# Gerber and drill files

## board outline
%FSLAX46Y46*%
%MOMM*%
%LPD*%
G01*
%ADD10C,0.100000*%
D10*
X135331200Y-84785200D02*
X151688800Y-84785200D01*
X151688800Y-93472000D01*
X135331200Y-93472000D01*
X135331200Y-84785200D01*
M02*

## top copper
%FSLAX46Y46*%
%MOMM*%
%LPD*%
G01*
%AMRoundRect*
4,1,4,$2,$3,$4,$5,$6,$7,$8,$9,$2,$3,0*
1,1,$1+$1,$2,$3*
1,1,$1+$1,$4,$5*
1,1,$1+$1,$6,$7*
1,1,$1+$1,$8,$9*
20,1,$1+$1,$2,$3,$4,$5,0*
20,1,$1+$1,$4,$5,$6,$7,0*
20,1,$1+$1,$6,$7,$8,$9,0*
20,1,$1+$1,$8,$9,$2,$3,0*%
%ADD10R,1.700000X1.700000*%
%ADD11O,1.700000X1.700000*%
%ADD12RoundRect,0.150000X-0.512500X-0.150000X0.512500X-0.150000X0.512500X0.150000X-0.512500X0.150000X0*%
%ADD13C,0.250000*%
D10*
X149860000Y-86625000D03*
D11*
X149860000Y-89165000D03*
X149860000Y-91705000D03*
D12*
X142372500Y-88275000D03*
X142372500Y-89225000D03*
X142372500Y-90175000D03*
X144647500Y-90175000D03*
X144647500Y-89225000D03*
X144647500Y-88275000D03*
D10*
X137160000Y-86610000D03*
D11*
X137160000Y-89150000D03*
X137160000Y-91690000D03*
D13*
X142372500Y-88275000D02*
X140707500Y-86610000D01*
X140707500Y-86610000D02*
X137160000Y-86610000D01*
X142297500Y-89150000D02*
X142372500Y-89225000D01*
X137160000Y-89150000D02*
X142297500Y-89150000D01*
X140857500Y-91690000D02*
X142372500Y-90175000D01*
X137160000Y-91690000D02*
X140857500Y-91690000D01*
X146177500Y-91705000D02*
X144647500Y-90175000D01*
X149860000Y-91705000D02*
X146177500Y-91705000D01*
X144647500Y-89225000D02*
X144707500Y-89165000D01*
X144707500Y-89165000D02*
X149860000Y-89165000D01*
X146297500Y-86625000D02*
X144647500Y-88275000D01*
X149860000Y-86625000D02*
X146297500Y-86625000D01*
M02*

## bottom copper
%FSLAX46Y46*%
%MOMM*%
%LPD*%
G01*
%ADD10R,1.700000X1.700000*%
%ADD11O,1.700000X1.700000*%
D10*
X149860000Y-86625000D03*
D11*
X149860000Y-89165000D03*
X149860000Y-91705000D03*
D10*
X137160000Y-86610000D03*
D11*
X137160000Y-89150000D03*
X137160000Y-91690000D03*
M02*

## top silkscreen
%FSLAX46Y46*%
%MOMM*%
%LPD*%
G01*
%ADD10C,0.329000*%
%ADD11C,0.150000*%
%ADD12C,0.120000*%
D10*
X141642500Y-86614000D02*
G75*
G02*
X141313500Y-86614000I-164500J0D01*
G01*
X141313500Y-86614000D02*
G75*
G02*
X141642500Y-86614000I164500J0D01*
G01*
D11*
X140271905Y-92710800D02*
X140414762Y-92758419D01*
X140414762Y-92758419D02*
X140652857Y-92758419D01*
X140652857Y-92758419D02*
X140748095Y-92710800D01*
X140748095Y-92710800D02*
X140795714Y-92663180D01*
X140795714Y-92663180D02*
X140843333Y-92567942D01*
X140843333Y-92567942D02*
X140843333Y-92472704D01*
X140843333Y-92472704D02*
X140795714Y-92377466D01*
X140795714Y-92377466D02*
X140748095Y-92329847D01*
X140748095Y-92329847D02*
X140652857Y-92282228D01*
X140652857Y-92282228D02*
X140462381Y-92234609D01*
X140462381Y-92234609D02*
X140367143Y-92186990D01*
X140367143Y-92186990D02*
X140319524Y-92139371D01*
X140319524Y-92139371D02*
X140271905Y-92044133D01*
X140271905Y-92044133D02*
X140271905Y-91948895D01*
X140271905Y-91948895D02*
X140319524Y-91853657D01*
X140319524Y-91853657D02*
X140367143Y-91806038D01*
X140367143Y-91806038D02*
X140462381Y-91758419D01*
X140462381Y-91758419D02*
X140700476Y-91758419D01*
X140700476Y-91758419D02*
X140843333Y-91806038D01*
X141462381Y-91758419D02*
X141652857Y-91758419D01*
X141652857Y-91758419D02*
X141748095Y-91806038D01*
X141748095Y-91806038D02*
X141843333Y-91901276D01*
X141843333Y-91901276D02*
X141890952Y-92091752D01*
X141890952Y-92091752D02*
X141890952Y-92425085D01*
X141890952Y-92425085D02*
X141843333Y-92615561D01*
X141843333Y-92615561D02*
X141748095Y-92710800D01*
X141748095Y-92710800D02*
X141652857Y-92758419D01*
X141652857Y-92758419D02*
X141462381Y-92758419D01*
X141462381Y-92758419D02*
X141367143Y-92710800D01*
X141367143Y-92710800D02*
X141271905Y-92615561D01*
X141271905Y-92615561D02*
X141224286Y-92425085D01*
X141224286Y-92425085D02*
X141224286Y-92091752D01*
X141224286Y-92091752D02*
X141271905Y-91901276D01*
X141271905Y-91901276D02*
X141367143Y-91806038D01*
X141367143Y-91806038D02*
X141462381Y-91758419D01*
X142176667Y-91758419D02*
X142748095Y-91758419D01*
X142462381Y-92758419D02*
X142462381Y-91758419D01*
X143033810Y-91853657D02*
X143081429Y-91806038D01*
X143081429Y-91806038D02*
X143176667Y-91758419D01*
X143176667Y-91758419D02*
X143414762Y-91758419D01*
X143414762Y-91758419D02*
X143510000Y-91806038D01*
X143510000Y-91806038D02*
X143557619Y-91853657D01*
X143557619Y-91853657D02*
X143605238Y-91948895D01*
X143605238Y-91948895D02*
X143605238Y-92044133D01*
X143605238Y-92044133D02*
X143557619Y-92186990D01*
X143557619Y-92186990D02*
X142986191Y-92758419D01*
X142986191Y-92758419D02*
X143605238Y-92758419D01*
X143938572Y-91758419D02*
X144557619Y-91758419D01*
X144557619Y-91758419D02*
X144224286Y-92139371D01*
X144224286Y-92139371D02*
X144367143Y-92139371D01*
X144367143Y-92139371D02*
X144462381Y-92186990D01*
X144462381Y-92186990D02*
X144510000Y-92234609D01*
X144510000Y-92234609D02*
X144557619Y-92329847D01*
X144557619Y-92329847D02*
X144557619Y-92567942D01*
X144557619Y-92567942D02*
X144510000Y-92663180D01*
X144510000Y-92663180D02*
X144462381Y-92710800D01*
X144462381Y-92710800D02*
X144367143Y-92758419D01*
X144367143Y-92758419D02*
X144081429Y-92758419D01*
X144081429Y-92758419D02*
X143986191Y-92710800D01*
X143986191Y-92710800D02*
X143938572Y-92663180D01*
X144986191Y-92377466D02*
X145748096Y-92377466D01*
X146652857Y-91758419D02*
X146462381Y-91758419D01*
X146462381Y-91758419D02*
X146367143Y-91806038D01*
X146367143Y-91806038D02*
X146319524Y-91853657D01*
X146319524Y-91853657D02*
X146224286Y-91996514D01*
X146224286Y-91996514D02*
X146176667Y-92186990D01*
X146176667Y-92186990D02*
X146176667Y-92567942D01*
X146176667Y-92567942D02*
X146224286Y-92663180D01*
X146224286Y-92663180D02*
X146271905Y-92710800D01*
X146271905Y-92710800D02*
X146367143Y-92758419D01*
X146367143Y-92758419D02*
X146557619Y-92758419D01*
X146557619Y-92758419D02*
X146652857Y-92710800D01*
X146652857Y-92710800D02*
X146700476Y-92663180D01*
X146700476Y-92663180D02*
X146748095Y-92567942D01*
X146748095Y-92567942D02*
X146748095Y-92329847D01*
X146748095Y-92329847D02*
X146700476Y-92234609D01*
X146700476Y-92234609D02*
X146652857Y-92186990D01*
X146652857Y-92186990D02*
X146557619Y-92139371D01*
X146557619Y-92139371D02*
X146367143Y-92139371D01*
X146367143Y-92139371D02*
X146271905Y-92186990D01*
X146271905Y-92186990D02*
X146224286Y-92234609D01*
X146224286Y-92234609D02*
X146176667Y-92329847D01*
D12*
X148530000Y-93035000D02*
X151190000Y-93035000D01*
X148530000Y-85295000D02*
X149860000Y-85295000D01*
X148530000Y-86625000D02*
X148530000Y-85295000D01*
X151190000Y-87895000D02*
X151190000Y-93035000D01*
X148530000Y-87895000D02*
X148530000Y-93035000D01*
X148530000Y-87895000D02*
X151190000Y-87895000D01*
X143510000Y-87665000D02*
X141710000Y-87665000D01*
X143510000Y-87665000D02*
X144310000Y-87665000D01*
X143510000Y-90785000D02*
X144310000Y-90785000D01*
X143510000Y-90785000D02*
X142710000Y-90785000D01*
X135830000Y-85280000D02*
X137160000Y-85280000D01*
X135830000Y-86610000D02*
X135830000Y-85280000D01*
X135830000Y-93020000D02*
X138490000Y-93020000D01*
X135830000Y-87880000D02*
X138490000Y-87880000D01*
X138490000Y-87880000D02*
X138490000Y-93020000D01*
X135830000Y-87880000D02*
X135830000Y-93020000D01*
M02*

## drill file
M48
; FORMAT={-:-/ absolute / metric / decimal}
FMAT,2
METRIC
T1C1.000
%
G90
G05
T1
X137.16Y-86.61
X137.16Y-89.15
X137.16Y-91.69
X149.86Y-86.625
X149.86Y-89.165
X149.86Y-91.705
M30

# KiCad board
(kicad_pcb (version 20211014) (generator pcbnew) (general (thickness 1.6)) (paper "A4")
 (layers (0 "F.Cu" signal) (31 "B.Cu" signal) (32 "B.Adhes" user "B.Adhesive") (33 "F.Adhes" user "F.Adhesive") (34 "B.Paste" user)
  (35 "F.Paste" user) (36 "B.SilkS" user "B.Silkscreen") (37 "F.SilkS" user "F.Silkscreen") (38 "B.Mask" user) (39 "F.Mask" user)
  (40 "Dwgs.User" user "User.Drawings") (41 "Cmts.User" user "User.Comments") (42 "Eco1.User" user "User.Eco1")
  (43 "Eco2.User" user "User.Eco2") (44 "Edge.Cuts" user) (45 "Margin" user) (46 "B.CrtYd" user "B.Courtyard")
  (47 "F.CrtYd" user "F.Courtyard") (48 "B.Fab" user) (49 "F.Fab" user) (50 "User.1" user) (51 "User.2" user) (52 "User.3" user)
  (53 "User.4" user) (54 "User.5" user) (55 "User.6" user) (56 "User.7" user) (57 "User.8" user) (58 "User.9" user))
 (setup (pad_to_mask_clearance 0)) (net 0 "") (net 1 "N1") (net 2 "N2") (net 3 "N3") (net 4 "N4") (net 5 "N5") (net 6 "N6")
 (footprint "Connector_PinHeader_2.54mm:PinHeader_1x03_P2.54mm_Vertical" (layer "F.Cu") (at 149.86 86.625)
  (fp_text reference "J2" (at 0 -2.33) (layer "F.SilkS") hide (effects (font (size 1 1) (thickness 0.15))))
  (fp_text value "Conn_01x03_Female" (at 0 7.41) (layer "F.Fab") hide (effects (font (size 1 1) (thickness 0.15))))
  (fp_line (start -1.33 6.41) (end 1.33 6.41) (layer "F.SilkS") (width 0.12))
  (fp_line (start -1.33 -1.33) (end 0 -1.33) (layer "F.SilkS") (width 0.12))
  (fp_line (start -1.33 0) (end -1.33 -1.33) (layer "F.SilkS") (width 0.12))
  (fp_line (start 1.33 1.27) (end 1.33 6.41) (layer "F.SilkS") (width 0.12))
  (fp_line (start -1.33 1.27) (end -1.33 6.41) (layer "F.SilkS") (width 0.12))
  (fp_line (start -1.33 1.27) (end 1.33 1.27) (layer "F.SilkS") (width 0.12))
  (pad "1" thru_hole rect (at 0 0) (size 1.7 1.7) (drill 1) (layers *.Cu *.Mask) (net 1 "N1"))
  (pad "2" thru_hole oval (at 0 2.54) (size 1.7 1.7) (drill 1) (layers *.Cu *.Mask) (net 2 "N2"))
  (pad "3" thru_hole oval (at 0 5.08) (size 1.7 1.7) (drill 1) (layers *.Cu *.Mask) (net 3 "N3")))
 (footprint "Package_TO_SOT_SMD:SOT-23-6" (layer "F.Cu") (at 143.51 89.225)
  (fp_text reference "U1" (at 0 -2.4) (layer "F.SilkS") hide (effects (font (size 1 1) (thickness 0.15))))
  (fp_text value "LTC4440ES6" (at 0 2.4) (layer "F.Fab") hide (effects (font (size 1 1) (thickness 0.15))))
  (fp_line (start 0 -1.56) (end -1.8 -1.56) (layer "F.SilkS") (width 0.12))
  (fp_line (start 0 -1.56) (end 0.8 -1.56) (layer "F.SilkS") (width 0.12))
  (fp_line (start 0 1.56) (end 0.8 1.56) (layer "F.SilkS") (width 0.12))
  (fp_line (start 0 1.56) (end -0.8 1.56) (layer "F.SilkS") (width 0.12))
  (pad "1" smd roundrect (at -1.1375 -0.95) (size 1.325 0.6) (layers "F.Cu" "F.Paste" "F.Mask") (roundrect_rratio 0.25) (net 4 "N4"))
  (pad "2" smd roundrect (at -1.1375 0) (size 1.325 0.6) (layers "F.Cu" "F.Paste" "F.Mask") (roundrect_rratio 0.25) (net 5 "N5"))
  (pad "3" smd roundrect (at -1.1375 0.95) (size 1.325 0.6) (layers "F.Cu" "F.Paste" "F.Mask") (roundrect_rratio 0.25) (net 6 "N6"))
  (pad "4" smd roundrect (at 1.1375 0.95) (size 1.325 0.6) (layers "F.Cu" "F.Paste" "F.Mask") (roundrect_rratio 0.25) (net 3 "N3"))
  (pad "5" smd roundrect (at 1.1375 0) (size 1.325 0.6) (layers "F.Cu" "F.Paste" "F.Mask") (roundrect_rratio 0.25) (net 2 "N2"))
  (pad "6" smd roundrect (at 1.1375 -0.95) (size 1.325 0.6) (layers "F.Cu" "F.Paste" "F.Mask") (roundrect_rratio 0.25) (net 1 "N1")))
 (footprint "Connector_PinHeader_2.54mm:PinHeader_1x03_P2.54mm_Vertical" (layer "F.Cu") (at 137.16 86.61)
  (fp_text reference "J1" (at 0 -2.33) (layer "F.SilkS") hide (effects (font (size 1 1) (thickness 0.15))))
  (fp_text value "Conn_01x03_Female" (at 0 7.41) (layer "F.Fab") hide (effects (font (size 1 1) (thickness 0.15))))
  (fp_line (start -1.33 -1.33) (end 0 -1.33) (layer "F.SilkS") (width 0.12))
  (fp_line (start -1.33 0) (end -1.33 -1.33) (layer "F.SilkS") (width 0.12))
  (fp_line (start -1.33 6.41) (end 1.33 6.41) (layer "F.SilkS") (width 0.12))
  (fp_line (start -1.33 1.27) (end 1.33 1.27) (layer "F.SilkS") (width 0.12))
  (fp_line (start 1.33 1.27) (end 1.33 6.41) (layer "F.SilkS") (width 0.12))
  (fp_line (start -1.33 1.27) (end -1.33 6.41) (layer "F.SilkS") (width 0.12))
  (pad "1" thru_hole rect (at 0 0) (size 1.7 1.7) (drill 1) (layers *.Cu *.Mask) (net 4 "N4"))
  (pad "2" thru_hole oval (at 0 2.54) (size 1.7 1.7) (drill 1) (layers *.Cu *.Mask) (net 5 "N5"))
  (pad "3" thru_hole oval (at 0 5.08) (size 1.7 1.7) (drill 1) (layers *.Cu *.Mask) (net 6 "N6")))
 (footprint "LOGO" (layer "B.Cu") (at 140.9 87 180)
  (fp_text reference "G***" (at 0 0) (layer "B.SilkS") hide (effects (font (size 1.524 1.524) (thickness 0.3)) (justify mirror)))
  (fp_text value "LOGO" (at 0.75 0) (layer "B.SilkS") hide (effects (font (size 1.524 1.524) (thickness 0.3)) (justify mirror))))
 (gr_circle (center 141.478 86.614) (end 141.732 86.614) (layer "F.SilkS") (width 0.15) (fill solid))
 (gr_rect (start 135.3312 84.7852) (end 151.6888 93.472) (layer "Edge.Cuts") (width 0.1) (fill none))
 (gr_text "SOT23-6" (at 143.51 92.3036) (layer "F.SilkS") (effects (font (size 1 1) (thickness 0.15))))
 (segment (start 142.3725 88.275) (end 140.7075 86.61) (width 0.25) (layer "F.Cu") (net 4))
 (segment (start 140.7075 86.61) (end 137.16 86.61) (width 0.25) (layer "F.Cu") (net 4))
 (segment (start 142.2975 89.15) (end 142.3725 89.225) (width 0.25) (layer "F.Cu") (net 5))
 (segment (start 137.16 89.15) (end 142.2975 89.15) (width 0.25) (layer "F.Cu") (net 5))
 (segment (start 140.8575 91.69) (end 142.3725 90.175) (width 0.25) (layer "F.Cu") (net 6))
 (segment (start 137.16 91.69) (end 140.8575 91.69) (width 0.25) (layer "F.Cu") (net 6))
 (segment (start 146.1775 91.705) (end 144.6475 90.175) (width 0.25) (layer "F.Cu") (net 3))
 (segment (start 149.86 91.705) (end 146.1775 91.705) (width 0.25) (layer "F.Cu") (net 3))
 (segment (start 144.6475 89.225) (end 144.7075 89.165) (width 0.25) (layer "F.Cu") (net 2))
 (segment (start 144.7075 89.165) (end 149.86 89.165) (width 0.25) (layer "F.Cu") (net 2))
 (segment (start 146.2975 86.625) (end 144.6475 88.275) (width 0.25) (layer "F.Cu") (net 1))
 (segment (start 149.86 86.625) (end 146.2975 86.625) (width 0.25) (layer "F.Cu") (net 1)))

